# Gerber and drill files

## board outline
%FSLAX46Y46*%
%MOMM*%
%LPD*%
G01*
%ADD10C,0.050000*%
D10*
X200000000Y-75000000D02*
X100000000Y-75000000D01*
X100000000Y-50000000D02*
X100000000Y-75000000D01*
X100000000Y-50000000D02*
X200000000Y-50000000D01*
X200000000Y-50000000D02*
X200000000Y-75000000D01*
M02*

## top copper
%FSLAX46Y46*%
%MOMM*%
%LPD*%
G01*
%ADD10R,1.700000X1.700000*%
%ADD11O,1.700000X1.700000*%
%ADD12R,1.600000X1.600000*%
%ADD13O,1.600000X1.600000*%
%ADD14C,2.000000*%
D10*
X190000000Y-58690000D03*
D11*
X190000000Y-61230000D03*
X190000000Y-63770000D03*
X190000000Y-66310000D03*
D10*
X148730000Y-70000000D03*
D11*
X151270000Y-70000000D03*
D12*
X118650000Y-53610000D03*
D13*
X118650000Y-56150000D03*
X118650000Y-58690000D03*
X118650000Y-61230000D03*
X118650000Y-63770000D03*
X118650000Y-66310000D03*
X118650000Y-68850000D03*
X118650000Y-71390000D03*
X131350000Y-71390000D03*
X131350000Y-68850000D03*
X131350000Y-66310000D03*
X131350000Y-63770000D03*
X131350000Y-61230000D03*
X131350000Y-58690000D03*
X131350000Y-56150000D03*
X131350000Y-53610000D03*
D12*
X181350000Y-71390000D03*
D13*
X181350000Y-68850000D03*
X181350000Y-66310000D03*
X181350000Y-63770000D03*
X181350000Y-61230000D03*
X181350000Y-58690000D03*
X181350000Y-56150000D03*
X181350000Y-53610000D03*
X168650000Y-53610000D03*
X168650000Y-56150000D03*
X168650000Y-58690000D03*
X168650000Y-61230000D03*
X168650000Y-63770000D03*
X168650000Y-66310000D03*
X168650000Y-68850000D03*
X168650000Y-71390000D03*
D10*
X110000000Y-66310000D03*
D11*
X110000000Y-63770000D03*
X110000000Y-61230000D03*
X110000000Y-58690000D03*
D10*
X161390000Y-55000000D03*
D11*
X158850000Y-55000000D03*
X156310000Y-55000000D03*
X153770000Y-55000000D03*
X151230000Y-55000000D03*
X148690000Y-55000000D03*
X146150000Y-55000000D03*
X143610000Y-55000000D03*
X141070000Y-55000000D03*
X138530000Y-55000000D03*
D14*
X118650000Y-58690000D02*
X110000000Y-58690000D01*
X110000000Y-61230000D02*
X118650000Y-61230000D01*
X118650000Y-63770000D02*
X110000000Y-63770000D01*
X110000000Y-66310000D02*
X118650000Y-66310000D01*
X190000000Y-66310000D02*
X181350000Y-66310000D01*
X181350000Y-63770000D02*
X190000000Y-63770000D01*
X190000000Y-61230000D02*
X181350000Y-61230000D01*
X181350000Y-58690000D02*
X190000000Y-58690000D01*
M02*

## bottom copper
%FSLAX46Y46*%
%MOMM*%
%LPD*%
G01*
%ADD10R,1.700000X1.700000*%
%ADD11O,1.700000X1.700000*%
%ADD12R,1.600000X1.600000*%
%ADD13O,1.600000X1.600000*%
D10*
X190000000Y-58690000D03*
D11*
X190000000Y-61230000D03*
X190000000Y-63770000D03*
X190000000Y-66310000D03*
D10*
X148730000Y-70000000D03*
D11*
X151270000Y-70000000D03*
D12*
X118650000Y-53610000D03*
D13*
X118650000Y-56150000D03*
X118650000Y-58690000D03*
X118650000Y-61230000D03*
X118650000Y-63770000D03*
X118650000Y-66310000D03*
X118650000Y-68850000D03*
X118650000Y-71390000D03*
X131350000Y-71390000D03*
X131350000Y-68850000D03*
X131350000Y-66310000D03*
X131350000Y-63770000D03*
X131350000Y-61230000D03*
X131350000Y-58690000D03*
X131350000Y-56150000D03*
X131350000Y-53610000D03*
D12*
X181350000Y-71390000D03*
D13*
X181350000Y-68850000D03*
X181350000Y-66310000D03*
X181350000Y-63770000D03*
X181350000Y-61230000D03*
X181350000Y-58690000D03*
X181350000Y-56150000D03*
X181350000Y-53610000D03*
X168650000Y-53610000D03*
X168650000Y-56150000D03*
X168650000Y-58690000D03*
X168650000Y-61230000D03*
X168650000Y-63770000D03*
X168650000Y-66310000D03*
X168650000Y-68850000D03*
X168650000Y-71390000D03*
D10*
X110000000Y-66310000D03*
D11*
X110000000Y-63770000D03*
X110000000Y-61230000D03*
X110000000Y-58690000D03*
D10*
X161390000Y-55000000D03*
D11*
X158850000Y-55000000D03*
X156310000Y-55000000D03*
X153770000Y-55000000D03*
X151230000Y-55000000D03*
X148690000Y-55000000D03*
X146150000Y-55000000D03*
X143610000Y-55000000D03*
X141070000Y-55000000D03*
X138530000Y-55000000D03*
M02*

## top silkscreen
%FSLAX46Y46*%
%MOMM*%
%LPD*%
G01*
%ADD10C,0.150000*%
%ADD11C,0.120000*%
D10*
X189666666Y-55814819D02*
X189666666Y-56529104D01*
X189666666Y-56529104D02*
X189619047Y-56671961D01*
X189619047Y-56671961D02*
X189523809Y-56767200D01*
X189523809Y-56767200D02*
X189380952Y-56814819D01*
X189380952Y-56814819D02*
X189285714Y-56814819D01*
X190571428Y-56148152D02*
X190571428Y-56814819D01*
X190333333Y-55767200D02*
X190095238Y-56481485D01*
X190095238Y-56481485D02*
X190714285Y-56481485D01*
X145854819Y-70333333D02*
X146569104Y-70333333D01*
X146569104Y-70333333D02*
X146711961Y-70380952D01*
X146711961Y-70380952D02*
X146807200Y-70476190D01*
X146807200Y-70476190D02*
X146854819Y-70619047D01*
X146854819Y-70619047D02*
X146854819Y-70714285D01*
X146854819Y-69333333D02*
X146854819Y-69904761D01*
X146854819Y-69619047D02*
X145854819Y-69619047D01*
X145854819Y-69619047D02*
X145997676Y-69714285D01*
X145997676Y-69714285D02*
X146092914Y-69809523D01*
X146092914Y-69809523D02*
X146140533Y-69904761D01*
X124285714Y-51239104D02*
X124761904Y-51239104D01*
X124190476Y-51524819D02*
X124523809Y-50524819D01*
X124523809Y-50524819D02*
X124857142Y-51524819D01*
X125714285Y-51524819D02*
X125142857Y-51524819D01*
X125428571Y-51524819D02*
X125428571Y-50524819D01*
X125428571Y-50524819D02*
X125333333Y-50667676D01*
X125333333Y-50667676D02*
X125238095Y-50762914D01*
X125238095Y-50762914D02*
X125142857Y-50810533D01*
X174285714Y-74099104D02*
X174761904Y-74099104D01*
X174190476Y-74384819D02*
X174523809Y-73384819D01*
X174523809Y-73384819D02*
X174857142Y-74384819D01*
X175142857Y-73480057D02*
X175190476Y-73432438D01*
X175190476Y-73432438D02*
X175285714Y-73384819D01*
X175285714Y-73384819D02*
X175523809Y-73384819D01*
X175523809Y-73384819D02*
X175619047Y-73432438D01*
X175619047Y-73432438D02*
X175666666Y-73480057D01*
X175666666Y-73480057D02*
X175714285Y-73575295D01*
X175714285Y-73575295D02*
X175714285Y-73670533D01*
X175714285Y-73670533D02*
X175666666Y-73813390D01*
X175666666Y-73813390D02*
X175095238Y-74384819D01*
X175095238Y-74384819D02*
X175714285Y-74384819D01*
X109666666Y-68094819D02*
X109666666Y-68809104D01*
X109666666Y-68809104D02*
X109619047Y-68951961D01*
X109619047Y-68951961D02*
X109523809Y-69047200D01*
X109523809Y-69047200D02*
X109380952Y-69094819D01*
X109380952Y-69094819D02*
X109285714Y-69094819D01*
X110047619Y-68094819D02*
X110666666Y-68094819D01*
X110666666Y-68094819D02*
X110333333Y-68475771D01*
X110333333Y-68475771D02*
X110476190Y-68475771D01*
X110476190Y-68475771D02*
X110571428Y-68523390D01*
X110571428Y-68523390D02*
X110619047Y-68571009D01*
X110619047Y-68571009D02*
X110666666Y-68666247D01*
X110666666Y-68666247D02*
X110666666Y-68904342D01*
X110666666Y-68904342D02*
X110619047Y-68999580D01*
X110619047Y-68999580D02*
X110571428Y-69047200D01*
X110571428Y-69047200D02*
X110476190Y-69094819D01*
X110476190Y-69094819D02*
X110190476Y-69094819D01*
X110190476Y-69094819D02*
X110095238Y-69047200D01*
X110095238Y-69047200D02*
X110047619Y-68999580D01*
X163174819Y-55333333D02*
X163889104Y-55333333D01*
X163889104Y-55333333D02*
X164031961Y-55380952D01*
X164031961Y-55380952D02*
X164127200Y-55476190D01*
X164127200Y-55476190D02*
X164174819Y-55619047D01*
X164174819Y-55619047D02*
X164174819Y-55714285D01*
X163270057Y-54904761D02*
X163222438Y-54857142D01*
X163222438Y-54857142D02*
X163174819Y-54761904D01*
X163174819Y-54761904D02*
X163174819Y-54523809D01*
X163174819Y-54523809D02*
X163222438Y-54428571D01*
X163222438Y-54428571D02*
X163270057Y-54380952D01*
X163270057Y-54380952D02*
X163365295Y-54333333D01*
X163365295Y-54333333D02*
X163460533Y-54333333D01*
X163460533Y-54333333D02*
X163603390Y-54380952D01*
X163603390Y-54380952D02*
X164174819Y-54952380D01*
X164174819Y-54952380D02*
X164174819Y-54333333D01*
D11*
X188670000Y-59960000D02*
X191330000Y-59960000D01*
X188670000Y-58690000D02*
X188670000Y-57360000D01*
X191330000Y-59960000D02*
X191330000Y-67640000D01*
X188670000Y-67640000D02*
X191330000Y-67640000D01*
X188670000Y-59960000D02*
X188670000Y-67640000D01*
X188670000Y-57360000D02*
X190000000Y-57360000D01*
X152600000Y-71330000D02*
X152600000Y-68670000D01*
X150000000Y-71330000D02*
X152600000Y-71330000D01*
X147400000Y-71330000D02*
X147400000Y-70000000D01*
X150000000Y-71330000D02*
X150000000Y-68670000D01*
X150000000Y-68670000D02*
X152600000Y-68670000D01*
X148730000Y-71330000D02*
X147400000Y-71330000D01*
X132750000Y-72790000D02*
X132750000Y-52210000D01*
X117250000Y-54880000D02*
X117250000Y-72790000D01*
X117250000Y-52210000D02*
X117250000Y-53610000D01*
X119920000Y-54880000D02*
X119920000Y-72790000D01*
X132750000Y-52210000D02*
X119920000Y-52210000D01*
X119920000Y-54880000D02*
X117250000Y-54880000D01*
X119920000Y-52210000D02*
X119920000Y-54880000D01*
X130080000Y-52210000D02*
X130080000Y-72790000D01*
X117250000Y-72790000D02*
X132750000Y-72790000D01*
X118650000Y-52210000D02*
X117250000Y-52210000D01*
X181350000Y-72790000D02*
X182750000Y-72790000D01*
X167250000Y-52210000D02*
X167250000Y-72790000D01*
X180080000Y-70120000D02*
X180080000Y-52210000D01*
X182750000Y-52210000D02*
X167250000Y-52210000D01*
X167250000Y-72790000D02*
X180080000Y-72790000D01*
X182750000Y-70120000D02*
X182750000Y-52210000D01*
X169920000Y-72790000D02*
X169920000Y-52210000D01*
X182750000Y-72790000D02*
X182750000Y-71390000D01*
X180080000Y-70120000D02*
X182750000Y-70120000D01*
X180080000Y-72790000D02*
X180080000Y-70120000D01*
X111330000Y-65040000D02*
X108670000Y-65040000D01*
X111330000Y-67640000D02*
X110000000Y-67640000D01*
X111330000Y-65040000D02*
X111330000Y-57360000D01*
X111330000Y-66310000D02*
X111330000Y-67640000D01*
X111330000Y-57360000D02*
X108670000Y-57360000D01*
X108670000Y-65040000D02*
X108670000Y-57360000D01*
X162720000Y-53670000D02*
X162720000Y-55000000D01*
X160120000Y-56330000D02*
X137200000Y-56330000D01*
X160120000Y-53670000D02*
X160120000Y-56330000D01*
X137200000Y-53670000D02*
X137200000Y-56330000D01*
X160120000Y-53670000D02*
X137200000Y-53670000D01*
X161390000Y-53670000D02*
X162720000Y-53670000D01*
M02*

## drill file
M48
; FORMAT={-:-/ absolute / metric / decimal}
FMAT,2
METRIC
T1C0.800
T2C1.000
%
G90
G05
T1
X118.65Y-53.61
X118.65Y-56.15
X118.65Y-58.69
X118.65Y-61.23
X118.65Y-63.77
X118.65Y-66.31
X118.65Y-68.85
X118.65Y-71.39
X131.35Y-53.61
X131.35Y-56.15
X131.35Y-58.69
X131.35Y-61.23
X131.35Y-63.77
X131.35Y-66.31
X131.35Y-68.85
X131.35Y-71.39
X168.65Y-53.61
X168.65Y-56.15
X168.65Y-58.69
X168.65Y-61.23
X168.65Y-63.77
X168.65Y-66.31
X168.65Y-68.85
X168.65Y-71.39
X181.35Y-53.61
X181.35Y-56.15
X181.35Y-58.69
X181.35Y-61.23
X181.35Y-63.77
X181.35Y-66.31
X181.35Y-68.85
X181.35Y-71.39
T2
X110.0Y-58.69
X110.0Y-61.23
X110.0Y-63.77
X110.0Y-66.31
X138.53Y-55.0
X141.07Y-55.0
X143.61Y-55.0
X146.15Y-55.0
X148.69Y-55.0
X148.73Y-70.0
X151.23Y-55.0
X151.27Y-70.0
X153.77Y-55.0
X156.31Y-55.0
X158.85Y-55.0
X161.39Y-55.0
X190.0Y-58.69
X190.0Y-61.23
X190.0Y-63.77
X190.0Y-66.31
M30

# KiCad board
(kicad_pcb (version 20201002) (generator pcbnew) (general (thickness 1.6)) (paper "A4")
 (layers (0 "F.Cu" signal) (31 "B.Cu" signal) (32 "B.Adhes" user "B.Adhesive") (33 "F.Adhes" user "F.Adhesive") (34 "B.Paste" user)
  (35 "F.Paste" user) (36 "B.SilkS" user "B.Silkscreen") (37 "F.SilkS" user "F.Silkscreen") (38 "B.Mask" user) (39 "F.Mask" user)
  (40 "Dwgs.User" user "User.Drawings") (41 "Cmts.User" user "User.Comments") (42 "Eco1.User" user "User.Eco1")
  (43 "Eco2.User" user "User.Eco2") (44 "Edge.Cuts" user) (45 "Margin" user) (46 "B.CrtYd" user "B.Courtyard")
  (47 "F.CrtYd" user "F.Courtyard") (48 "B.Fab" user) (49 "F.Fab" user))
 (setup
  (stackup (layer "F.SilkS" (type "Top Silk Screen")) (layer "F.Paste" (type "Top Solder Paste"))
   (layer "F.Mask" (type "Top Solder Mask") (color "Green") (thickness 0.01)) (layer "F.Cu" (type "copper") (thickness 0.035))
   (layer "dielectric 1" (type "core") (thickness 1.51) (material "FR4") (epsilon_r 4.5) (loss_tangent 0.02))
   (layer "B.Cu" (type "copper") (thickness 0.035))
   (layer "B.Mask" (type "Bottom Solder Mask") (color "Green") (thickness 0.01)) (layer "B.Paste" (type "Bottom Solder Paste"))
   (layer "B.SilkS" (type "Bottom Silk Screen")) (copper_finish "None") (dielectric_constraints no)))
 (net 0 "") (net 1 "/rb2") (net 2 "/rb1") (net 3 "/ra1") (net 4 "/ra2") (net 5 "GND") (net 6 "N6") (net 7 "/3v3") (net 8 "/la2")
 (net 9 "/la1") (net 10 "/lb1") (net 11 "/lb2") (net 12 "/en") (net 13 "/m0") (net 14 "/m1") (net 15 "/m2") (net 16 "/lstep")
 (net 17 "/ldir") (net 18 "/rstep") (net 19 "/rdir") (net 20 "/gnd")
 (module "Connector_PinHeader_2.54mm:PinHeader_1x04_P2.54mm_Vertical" (layer "F.Cu") (at 190 58.69)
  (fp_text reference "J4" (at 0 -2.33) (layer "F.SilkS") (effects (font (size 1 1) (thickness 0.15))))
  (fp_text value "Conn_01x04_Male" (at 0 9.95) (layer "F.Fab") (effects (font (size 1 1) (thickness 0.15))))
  (fp_line (start -1.33 1.27) (end 1.33 1.27) (layer "F.SilkS") (width 0.12))
  (fp_line (start -1.33 0) (end -1.33 -1.33) (layer "F.SilkS") (width 0.12))
  (fp_line (start 1.33 1.27) (end 1.33 8.95) (layer "F.SilkS") (width 0.12))
  (fp_line (start -1.33 8.95) (end 1.33 8.95) (layer "F.SilkS") (width 0.12))
  (fp_line (start -1.33 1.27) (end -1.33 8.95) (layer "F.SilkS") (width 0.12))
  (fp_line (start -1.33 -1.33) (end 0 -1.33) (layer "F.SilkS") (width 0.12))
  (pad "1" thru_hole rect (at 0 0) (size 1.7 1.7) (drill 1) (layers *.Cu *.Mask) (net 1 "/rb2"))
  (pad "2" thru_hole oval (at 0 2.54) (size 1.7 1.7) (drill 1) (layers *.Cu *.Mask) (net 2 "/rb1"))
  (pad "3" thru_hole oval (at 0 5.08) (size 1.7 1.7) (drill 1) (layers *.Cu *.Mask) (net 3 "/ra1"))
  (pad "4" thru_hole oval (at 0 7.62) (size 1.7 1.7) (drill 1) (layers *.Cu *.Mask) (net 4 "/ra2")))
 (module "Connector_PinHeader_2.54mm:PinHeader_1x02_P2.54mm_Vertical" (layer "F.Cu") (at 148.73 70 90)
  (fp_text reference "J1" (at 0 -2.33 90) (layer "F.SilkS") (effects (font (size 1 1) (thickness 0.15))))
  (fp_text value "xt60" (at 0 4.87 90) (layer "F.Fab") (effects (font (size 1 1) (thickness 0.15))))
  (fp_line (start -1.33 3.87) (end 1.33 3.87) (layer "F.SilkS") (width 0.12))
  (fp_line (start -1.33 1.27) (end -1.33 3.87) (layer "F.SilkS") (width 0.12))
  (fp_line (start -1.33 -1.33) (end 0 -1.33) (layer "F.SilkS") (width 0.12))
  (fp_line (start -1.33 1.27) (end 1.33 1.27) (layer "F.SilkS") (width 0.12))
  (fp_line (start 1.33 1.27) (end 1.33 3.87) (layer "F.SilkS") (width 0.12))
  (fp_line (start -1.33 0) (end -1.33 -1.33) (layer "F.SilkS") (width 0.12))
  (pad "1" thru_hole rect (at 0 0 90) (size 1.7 1.7) (drill 1) (layers *.Cu *.Mask) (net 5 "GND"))
  (pad "2" thru_hole oval (at 0 2.54 90) (size 1.7 1.7) (drill 1) (layers *.Cu *.Mask) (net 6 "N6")))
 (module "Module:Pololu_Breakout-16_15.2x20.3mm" (layer "F.Cu") (at 118.65 53.61)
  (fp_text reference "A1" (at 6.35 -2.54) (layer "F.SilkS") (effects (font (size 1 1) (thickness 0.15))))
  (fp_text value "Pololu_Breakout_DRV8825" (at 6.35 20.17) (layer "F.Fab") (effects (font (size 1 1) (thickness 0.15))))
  (fp_line (start 14.1 19.18) (end 14.1 -1.4) (layer "F.SilkS") (width 0.12))
  (fp_line (start -1.4 1.27) (end -1.4 19.18) (layer "F.SilkS") (width 0.12))
  (fp_line (start -1.4 -1.4) (end -1.4 0) (layer "F.SilkS") (width 0.12))
  (fp_line (start 1.27 1.27) (end 1.27 19.18) (layer "F.SilkS") (width 0.12))
  (fp_line (start 14.1 -1.4) (end 1.27 -1.4) (layer "F.SilkS") (width 0.12))
  (fp_line (start 1.27 1.27) (end -1.4 1.27) (layer "F.SilkS") (width 0.12))
  (fp_line (start 1.27 -1.4) (end 1.27 1.27) (layer "F.SilkS") (width 0.12))
  (fp_line (start 11.43 -1.4) (end 11.43 19.18) (layer "F.SilkS") (width 0.12))
  (fp_line (start -1.4 19.18) (end 14.1 19.18) (layer "F.SilkS") (width 0.12))
  (fp_line (start 0 -1.4) (end -1.4 -1.4) (layer "F.SilkS") (width 0.12))
  (pad "1" thru_hole rect (at 0 0) (size 1.6 1.6) (drill 0.8) (layers *.Cu *.Mask) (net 5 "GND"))
  (pad "2" thru_hole oval (at 0 2.54) (size 1.6 1.6) (drill 0.8) (layers *.Cu *.Mask) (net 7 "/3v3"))
  (pad "3" thru_hole oval (at 0 5.08) (size 1.6 1.6) (drill 0.8) (layers *.Cu *.Mask) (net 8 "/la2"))
  (pad "4" thru_hole oval (at 0 7.62) (size 1.6 1.6) (drill 0.8) (layers *.Cu *.Mask) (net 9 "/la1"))
  (pad "5" thru_hole oval (at 0 10.16) (size 1.6 1.6) (drill 0.8) (layers *.Cu *.Mask) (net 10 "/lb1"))
  (pad "6" thru_hole oval (at 0 12.7) (size 1.6 1.6) (drill 0.8) (layers *.Cu *.Mask) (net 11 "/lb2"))
  (pad "7" thru_hole oval (at 0 15.24) (size 1.6 1.6) (drill 0.8) (layers *.Cu *.Mask) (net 5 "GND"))
  (pad "8" thru_hole oval (at 0 17.78) (size 1.6 1.6) (drill 0.8) (layers *.Cu *.Mask) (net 6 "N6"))
  (pad "9" thru_hole oval (at 12.7 17.78) (size 1.6 1.6) (drill 0.8) (layers *.Cu *.Mask) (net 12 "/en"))
  (pad "10" thru_hole oval (at 12.7 15.24) (size 1.6 1.6) (drill 0.8) (layers *.Cu *.Mask) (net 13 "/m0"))
  (pad "11" thru_hole oval (at 12.7 12.7) (size 1.6 1.6) (drill 0.8) (layers *.Cu *.Mask) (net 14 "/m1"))
  (pad "12" thru_hole oval (at 12.7 10.16) (size 1.6 1.6) (drill 0.8) (layers *.Cu *.Mask) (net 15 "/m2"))
  (pad "13" thru_hole oval (at 12.7 7.62) (size 1.6 1.6) (drill 0.8) (layers *.Cu *.Mask) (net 7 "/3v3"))
  (pad "14" thru_hole oval (at 12.7 5.08) (size 1.6 1.6) (drill 0.8) (layers *.Cu *.Mask) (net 7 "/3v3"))
  (pad "15" thru_hole oval (at 12.7 2.54) (size 1.6 1.6) (drill 0.8) (layers *.Cu *.Mask) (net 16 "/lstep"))
  (pad "16" thru_hole oval (at 12.7 0) (size 1.6 1.6) (drill 0.8) (layers *.Cu *.Mask) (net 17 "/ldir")))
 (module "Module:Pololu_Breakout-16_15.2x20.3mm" (layer "F.Cu") (at 181.35 71.39 180)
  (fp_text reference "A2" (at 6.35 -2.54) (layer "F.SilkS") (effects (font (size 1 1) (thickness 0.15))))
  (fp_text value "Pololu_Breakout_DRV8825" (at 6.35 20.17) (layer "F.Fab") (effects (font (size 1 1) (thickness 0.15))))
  (fp_line (start 0 -1.4) (end -1.4 -1.4) (layer "F.SilkS") (width 0.12))
  (fp_line (start 14.1 19.18) (end 14.1 -1.4) (layer "F.SilkS") (width 0.12))
  (fp_line (start 1.27 1.27) (end 1.27 19.18) (layer "F.SilkS") (width 0.12))
  (fp_line (start -1.4 19.18) (end 14.1 19.18) (layer "F.SilkS") (width 0.12))
  (fp_line (start 14.1 -1.4) (end 1.27 -1.4) (layer "F.SilkS") (width 0.12))
  (fp_line (start -1.4 1.27) (end -1.4 19.18) (layer "F.SilkS") (width 0.12))
  (fp_line (start 11.43 -1.4) (end 11.43 19.18) (layer "F.SilkS") (width 0.12))
  (fp_line (start -1.4 -1.4) (end -1.4 0) (layer "F.SilkS") (width 0.12))
  (fp_line (start 1.27 1.27) (end -1.4 1.27) (layer "F.SilkS") (width 0.12))
  (fp_line (start 1.27 -1.4) (end 1.27 1.27) (layer "F.SilkS") (width 0.12))
  (pad "1" thru_hole rect (at 0 0 180) (size 1.6 1.6) (drill 0.8) (layers *.Cu *.Mask) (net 5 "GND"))
  (pad "2" thru_hole oval (at 0 2.54 180) (size 1.6 1.6) (drill 0.8) (layers *.Cu *.Mask) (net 7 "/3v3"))
  (pad "3" thru_hole oval (at 0 5.08 180) (size 1.6 1.6) (drill 0.8) (layers *.Cu *.Mask) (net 4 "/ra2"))
  (pad "4" thru_hole oval (at 0 7.62 180) (size 1.6 1.6) (drill 0.8) (layers *.Cu *.Mask) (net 3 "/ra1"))
  (pad "5" thru_hole oval (at 0 10.16 180) (size 1.6 1.6) (drill 0.8) (layers *.Cu *.Mask) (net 2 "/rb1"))
  (pad "6" thru_hole oval (at 0 12.7 180) (size 1.6 1.6) (drill 0.8) (layers *.Cu *.Mask) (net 1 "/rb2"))
  (pad "7" thru_hole oval (at 0 15.24 180) (size 1.6 1.6) (drill 0.8) (layers *.Cu *.Mask) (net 5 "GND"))
  (pad "8" thru_hole oval (at 0 17.78 180) (size 1.6 1.6) (drill 0.8) (layers *.Cu *.Mask) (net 6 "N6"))
  (pad "9" thru_hole oval (at 12.7 17.78 180) (size 1.6 1.6) (drill 0.8) (layers *.Cu *.Mask) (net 12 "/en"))
  (pad "10" thru_hole oval (at 12.7 15.24 180) (size 1.6 1.6) (drill 0.8) (layers *.Cu *.Mask) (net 13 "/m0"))
  (pad "11" thru_hole oval (at 12.7 12.7 180) (size 1.6 1.6) (drill 0.8) (layers *.Cu *.Mask) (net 14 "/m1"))
  (pad "12" thru_hole oval (at 12.7 10.16 180) (size 1.6 1.6) (drill 0.8) (layers *.Cu *.Mask) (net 15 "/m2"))
  (pad "13" thru_hole oval (at 12.7 7.62 180) (size 1.6 1.6) (drill 0.8) (layers *.Cu *.Mask) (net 7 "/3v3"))
  (pad "14" thru_hole oval (at 12.7 5.08 180) (size 1.6 1.6) (drill 0.8) (layers *.Cu *.Mask) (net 7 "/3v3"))
  (pad "15" thru_hole oval (at 12.7 2.54 180) (size 1.6 1.6) (drill 0.8) (layers *.Cu *.Mask) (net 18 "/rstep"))
  (pad "16" thru_hole oval (at 12.7 0 180) (size 1.6 1.6) (drill 0.8) (layers *.Cu *.Mask) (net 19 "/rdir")))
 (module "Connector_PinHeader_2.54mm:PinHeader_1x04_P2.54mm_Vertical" (layer "F.Cu") (at 110 66.31 180)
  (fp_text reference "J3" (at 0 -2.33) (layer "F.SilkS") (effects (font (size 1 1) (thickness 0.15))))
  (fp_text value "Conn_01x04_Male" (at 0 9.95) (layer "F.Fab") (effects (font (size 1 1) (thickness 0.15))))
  (fp_line (start -1.33 1.27) (end 1.33 1.27) (layer "F.SilkS") (width 0.12))
  (fp_line (start -1.33 -1.33) (end 0 -1.33) (layer "F.SilkS") (width 0.12))
  (fp_line (start -1.33 1.27) (end -1.33 8.95) (layer "F.SilkS") (width 0.12))
  (fp_line (start -1.33 0) (end -1.33 -1.33) (layer "F.SilkS") (width 0.12))
  (fp_line (start -1.33 8.95) (end 1.33 8.95) (layer "F.SilkS") (width 0.12))
  (fp_line (start 1.33 1.27) (end 1.33 8.95) (layer "F.SilkS") (width 0.12))
  (pad "1" thru_hole rect (at 0 0 180) (size 1.7 1.7) (drill 1) (layers *.Cu *.Mask) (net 11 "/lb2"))
  (pad "2" thru_hole oval (at 0 2.54 180) (size 1.7 1.7) (drill 1) (layers *.Cu *.Mask) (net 10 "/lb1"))
  (pad "3" thru_hole oval (at 0 5.08 180) (size 1.7 1.7) (drill 1) (layers *.Cu *.Mask) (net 9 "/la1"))
  (pad "4" thru_hole oval (at 0 7.62 180) (size 1.7 1.7) (drill 1) (layers *.Cu *.Mask) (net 8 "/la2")))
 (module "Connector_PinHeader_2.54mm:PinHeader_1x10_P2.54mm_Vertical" (layer "F.Cu") (at 161.39 55 -90)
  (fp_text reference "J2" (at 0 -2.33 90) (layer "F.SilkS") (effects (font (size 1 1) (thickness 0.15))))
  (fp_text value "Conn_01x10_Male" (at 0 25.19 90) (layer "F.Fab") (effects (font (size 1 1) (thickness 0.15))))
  (fp_line (start -1.33 -1.33) (end 0 -1.33) (layer "F.SilkS") (width 0.12))
  (fp_line (start 1.33 1.27) (end 1.33 24.19) (layer "F.SilkS") (width 0.12))
  (fp_line (start -1.33 1.27) (end 1.33 1.27) (layer "F.SilkS") (width 0.12))
  (fp_line (start -1.33 24.19) (end 1.33 24.19) (layer "F.SilkS") (width 0.12))
  (fp_line (start -1.33 1.27) (end -1.33 24.19) (layer "F.SilkS") (width 0.12))
  (fp_line (start -1.33 0) (end -1.33 -1.33) (layer "F.SilkS") (width 0.12))
  (pad "1" thru_hole rect (at 0 0 270) (size 1.7 1.7) (drill 1) (layers *.Cu *.Mask) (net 7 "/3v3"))
  (pad "2" thru_hole oval (at 0 2.54 270) (size 1.7 1.7) (drill 1) (layers *.Cu *.Mask) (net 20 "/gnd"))
  (pad "3" thru_hole oval (at 0 5.08 270) (size 1.7 1.7) (drill 1) (layers *.Cu *.Mask) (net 13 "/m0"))
  (pad "4" thru_hole oval (at 0 7.62 270) (size 1.7 1.7) (drill 1) (layers *.Cu *.Mask) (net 14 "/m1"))
  (pad "5" thru_hole oval (at 0 10.16 270) (size 1.7 1.7) (drill 1) (layers *.Cu *.Mask) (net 15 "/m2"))
  (pad "6" thru_hole oval (at 0 12.7 270) (size 1.7 1.7) (drill 1) (layers *.Cu *.Mask) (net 12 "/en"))
  (pad "7" thru_hole oval (at 0 15.24 270) (size 1.7 1.7) (drill 1) (layers *.Cu *.Mask) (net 17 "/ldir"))
  (pad "8" thru_hole oval (at 0 17.78 270) (size 1.7 1.7) (drill 1) (layers *.Cu *.Mask) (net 16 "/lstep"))
  (pad "9" thru_hole oval (at 0 20.32 270) (size 1.7 1.7) (drill 1) (layers *.Cu *.Mask) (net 19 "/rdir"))
  (pad "10" thru_hole oval (at 0 22.86 270) (size 1.7 1.7) (drill 1) (layers *.Cu *.Mask) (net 18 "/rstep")))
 (gr_line (start 200 75) (end 100 75) (layer "Edge.Cuts") (width 0.05))
 (gr_line (start 100 50) (end 100 75) (layer "Edge.Cuts") (width 0.05))
 (gr_line (start 100 50) (end 200 50) (layer "Edge.Cuts") (width 0.05))
 (gr_line (start 200 50) (end 200 75) (layer "Edge.Cuts") (width 0.05))
 (segment (start 118.65 58.69) (end 110 58.69) (width 2) (layer "F.Cu") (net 8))
 (segment (start 110 61.23) (end 118.65 61.23) (width 2) (layer "F.Cu") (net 9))
 (segment (start 118.65 63.77) (end 110 63.77) (width 2) (layer "F.Cu") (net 10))
 (segment (start 110 66.31) (end 118.65 66.31) (width 2) (layer "F.Cu") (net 11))
 (segment (start 190 66.31) (end 181.35 66.31) (width 2) (layer "F.Cu") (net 4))
 (segment (start 181.35 63.77) (end 190 63.77) (width 2) (layer "F.Cu") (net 3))
 (segment (start 190 61.23) (end 181.35 61.23) (width 2) (layer "F.Cu") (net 2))
 (segment (start 181.35 58.69) (end 190 58.69) (width 2) (layer "F.Cu") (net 1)))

